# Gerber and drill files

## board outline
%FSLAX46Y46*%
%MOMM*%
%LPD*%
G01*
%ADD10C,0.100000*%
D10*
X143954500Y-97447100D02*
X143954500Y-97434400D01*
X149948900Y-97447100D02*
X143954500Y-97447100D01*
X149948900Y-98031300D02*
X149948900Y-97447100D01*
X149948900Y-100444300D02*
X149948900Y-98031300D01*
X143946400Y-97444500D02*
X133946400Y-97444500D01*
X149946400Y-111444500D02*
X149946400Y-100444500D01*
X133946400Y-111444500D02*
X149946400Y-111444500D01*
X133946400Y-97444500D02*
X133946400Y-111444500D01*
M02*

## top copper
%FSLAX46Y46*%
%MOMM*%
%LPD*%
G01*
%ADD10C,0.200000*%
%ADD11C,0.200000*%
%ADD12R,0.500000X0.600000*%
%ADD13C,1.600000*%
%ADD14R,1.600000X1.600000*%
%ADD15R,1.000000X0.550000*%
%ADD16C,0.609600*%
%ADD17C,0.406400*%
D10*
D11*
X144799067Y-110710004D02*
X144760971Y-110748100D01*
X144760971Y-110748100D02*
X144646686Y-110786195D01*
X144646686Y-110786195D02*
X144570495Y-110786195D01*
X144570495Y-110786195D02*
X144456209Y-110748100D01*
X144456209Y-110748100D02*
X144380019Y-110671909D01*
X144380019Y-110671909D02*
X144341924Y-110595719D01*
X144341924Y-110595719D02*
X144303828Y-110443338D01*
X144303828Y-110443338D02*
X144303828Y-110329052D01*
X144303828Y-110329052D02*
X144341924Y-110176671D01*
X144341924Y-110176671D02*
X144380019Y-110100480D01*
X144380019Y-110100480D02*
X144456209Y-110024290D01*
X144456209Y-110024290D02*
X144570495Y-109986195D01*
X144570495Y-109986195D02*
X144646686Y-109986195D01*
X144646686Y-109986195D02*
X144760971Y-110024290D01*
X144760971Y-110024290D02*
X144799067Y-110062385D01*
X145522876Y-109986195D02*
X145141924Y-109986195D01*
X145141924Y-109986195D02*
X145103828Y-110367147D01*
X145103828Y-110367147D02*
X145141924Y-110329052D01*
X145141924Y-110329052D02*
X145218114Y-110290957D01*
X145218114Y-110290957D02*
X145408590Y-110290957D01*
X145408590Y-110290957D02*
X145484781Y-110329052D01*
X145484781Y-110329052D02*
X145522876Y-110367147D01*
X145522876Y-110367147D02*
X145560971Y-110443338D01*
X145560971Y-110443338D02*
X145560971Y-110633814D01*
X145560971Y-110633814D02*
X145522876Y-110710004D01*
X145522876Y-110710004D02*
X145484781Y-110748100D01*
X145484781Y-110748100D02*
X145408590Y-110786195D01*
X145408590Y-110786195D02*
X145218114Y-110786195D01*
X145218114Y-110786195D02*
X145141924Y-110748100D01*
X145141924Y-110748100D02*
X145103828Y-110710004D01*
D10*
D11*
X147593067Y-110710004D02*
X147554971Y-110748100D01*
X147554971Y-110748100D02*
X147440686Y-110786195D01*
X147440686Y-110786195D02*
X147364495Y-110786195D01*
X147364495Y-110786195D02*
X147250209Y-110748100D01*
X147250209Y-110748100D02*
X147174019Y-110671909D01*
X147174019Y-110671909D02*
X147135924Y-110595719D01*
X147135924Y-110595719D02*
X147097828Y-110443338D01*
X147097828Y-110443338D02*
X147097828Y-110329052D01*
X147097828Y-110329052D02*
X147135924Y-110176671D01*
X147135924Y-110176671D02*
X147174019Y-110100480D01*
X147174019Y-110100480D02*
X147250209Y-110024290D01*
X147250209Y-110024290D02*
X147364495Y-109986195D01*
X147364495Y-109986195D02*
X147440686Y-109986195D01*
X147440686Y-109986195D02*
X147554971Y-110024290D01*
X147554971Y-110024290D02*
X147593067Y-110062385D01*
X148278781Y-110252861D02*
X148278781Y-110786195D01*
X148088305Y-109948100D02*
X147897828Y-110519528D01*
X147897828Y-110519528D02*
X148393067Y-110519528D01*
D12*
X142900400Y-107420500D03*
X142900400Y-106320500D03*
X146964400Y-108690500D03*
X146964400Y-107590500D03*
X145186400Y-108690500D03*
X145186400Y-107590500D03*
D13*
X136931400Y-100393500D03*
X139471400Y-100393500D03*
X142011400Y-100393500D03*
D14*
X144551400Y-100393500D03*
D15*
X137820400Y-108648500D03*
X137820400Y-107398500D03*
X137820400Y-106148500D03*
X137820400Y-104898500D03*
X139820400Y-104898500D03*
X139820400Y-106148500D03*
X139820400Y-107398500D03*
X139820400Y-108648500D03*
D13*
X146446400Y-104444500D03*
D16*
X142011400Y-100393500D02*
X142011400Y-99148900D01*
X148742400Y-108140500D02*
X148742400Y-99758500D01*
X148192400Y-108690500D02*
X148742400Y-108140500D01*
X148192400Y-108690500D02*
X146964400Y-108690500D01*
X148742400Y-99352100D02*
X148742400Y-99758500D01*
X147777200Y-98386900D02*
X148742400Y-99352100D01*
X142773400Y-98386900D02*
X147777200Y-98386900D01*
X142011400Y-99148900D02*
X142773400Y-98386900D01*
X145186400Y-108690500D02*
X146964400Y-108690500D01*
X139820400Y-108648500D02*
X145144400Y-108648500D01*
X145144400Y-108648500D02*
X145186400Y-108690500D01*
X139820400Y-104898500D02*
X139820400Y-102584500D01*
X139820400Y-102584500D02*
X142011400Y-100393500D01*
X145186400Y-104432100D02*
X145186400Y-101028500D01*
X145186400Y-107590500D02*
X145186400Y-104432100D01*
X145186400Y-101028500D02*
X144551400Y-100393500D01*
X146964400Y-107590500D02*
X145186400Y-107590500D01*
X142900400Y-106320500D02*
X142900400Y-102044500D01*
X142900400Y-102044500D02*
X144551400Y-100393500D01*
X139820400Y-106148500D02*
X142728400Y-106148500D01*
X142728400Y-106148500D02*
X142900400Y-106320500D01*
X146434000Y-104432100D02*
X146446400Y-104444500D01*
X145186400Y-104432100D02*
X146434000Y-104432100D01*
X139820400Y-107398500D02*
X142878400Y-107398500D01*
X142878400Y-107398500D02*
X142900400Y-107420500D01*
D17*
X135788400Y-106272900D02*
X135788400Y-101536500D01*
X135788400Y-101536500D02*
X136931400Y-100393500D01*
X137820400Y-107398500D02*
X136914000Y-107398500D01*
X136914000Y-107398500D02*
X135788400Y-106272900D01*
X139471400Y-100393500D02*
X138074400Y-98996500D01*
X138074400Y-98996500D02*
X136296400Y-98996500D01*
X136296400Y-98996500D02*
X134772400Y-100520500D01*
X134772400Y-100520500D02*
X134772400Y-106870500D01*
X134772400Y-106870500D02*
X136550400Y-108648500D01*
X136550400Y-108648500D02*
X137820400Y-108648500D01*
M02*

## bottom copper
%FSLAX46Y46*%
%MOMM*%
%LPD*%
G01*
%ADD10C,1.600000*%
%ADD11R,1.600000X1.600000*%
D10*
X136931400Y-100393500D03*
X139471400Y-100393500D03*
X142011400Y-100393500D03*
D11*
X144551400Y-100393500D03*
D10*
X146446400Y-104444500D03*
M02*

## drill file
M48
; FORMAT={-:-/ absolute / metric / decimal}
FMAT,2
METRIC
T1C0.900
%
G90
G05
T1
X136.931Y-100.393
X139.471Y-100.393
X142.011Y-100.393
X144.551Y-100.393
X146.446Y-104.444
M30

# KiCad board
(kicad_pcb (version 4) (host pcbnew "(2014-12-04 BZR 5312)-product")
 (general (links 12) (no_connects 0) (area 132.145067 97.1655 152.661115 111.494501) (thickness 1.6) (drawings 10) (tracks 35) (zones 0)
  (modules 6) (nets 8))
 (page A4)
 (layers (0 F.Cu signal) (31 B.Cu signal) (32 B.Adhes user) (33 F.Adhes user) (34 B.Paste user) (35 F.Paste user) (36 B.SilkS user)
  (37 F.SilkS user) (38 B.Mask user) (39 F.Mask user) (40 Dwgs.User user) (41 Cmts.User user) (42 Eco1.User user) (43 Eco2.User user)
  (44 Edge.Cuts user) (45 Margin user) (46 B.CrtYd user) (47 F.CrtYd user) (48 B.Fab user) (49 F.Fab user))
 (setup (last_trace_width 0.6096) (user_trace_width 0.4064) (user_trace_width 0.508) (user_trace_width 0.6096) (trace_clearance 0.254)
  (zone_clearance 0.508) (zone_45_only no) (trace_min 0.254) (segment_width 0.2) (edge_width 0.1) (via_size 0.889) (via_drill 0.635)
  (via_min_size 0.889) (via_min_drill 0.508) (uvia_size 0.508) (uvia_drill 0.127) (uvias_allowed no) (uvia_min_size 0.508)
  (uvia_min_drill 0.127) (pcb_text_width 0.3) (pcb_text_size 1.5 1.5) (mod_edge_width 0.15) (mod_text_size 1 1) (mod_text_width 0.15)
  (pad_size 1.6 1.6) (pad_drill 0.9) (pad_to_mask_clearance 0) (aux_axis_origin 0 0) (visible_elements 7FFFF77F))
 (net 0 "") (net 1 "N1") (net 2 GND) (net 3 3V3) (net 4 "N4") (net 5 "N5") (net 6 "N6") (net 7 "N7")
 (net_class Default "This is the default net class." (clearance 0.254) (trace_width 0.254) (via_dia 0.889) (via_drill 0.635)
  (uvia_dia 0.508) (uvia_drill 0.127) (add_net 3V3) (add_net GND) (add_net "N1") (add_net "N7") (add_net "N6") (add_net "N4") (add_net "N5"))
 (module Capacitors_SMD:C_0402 (layer F.Cu) (at 142.9004 106.8705 90)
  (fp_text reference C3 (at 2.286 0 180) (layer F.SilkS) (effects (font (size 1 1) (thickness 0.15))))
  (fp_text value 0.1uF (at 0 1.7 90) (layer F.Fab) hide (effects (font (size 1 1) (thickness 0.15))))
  (pad 1 smd rect (at -0.55 0 90) (size 0.6 0.5) (layers F.Cu F.Paste F.Mask) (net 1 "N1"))
  (pad 2 smd rect (at 0.55 0 90) (size 0.6 0.5) (layers F.Cu F.Paste F.Mask) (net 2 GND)))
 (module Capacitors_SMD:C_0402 (layer F.Cu) (at 146.9644 108.1405 90)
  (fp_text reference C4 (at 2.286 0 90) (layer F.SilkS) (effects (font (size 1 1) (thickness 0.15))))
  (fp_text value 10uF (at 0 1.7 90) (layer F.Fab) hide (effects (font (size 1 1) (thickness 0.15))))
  (pad 1 smd rect (at -0.55 0 90) (size 0.6 0.5) (layers F.Cu F.Paste F.Mask) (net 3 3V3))
  (pad 2 smd rect (at 0.55 0 90) (size 0.6 0.5) (layers F.Cu F.Paste F.Mask) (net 2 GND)))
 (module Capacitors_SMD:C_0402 (layer F.Cu) (at 145.1864 108.1405 90)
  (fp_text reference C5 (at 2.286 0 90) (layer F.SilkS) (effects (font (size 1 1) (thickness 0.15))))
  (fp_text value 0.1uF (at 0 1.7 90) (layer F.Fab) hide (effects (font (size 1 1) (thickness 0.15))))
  (pad 1 smd rect (at -0.55 0 90) (size 0.6 0.5) (layers F.Cu F.Paste F.Mask) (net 3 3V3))
  (pad 2 smd rect (at 0.55 0 90) (size 0.6 0.5) (layers F.Cu F.Paste F.Mask) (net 2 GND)))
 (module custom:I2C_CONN (layer F.Cu) (at 142.0114 100.3935)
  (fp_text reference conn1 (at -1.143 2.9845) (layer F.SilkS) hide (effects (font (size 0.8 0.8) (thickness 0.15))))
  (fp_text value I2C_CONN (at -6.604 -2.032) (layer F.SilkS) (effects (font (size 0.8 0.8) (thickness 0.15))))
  (pad 1 thru_hole circle (at -5.08 0) (size 1.6 1.6) (drill 0.9) (layers *.Cu *.Mask F.SilkS) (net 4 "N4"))
  (pad 2 thru_hole circle (at -2.54 0) (size 1.6 1.6) (drill 0.9) (layers *.Cu *.Mask F.SilkS) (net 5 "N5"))
  (pad 3 thru_hole circle (at 0 0) (size 1.6 1.6) (drill 0.9) (layers *.Cu *.Mask F.SilkS) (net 3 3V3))
  (pad 4 thru_hole rect (at 2.54 0) (size 1.6 1.6) (drill 0.9) (layers *.Cu *.Mask F.SilkS) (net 2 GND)))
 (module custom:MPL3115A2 (layer F.Cu) (at 137.8204 108.6485 180)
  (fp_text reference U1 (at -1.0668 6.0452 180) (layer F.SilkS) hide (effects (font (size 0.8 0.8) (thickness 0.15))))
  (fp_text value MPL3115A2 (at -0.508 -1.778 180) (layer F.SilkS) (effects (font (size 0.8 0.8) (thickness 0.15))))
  (pad 8 smd rect (at 0 0 180) (size 1 0.55) (layers F.Cu F.Paste F.Mask) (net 5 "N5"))
  (pad 7 smd rect (at 0 1.25 180) (size 1 0.55) (layers F.Cu F.Paste F.Mask) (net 4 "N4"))
  (pad 6 smd rect (at 0 2.5 180) (size 1 0.55) (layers F.Cu F.Paste F.Mask) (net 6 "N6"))
  (pad 5 smd rect (at 0 3.75 180) (size 1 0.55) (layers F.Cu F.Paste F.Mask) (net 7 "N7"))
  (pad 4 smd rect (at -2 3.75 180) (size 1 0.55) (layers F.Cu F.Paste F.Mask) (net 3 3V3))
  (pad 3 smd rect (at -2 2.5 180) (size 1 0.55) (layers F.Cu F.Paste F.Mask) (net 2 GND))
  (pad 2 smd rect (at -2 1.25 180) (size 1 0.55) (layers F.Cu F.Paste F.Mask) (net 1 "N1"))
  (pad 1 smd rect (at -2 0 180) (size 1 0.55) (layers F.Cu F.Paste F.Mask) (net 3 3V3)))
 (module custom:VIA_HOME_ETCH (layer F.Cu) (at 146.4464 104.4445)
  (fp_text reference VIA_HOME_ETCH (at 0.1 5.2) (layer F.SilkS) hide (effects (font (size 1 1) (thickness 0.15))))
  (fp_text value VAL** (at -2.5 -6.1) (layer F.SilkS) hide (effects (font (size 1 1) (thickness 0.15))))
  (pad 1 thru_hole circle (at 0 0) (size 1.6 1.6) (drill 0.9) (layers *.Cu *.Mask F.SilkS) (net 2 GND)))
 (gr_line (start 143.9545 97.4471) (end 143.9545 97.4344) (angle 90) (layer Edge.Cuts) (width 0.1))
 (gr_line (start 149.9489 97.4471) (end 143.9545 97.4471) (angle 90) (layer Edge.Cuts) (width 0.1))
 (gr_line (start 149.9489 98.0313) (end 149.9489 97.4471) (angle 90) (layer Edge.Cuts) (width 0.1))
 (gr_line (start 149.9489 100.4443) (end 149.9489 98.0313) (angle 90) (layer Edge.Cuts) (width 0.1))
 (gr_line (start 143.9464 97.4445) (end 133.9464 97.4445) (angle 90) (layer Edge.Cuts) (width 0.1))
 (gr_line (start 149.9464 111.4445) (end 149.9464 100.4445) (angle 90) (layer Edge.Cuts) (width 0.1))
 (gr_line (start 133.9464 111.4445) (end 149.9464 111.4445) (angle 90) (layer Edge.Cuts) (width 0.1))
 (gr_line (start 133.9464 97.4445) (end 133.9464 111.4445) (angle 90) (layer Edge.Cuts) (width 0.1))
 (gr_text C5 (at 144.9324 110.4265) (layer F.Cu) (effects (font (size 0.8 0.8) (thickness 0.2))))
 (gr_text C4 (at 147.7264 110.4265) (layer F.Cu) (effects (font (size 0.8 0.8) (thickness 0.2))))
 (segment (start 142.0114 100.3935) (end 142.0114 99.1489) (width 0.6096) (layer F.Cu) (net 3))
 (segment (start 148.7424 108.1405) (end 148.7424 99.7585) (width 0.6096) (layer F.Cu) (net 3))
 (segment (start 148.1924 108.6905) (end 148.7424 108.1405) (width 0.6096) (layer F.Cu) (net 3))
 (segment (start 148.1924 108.6905) (end 146.9644 108.6905) (width 0.6096) (layer F.Cu) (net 3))
 (segment (start 148.7424 99.3521) (end 148.7424 99.7585) (width 0.6096) (layer F.Cu) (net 3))
 (segment (start 147.7772 98.3869) (end 148.7424 99.3521) (width 0.6096) (layer F.Cu) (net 3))
 (segment (start 142.7734 98.3869) (end 147.7772 98.3869) (width 0.6096) (layer F.Cu) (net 3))
 (segment (start 142.0114 99.1489) (end 142.7734 98.3869) (width 0.6096) (layer F.Cu) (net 3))
 (segment (start 145.1864 108.6905) (end 146.9644 108.6905) (width 0.6096) (layer F.Cu) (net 3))
 (segment (start 139.8204 108.6485) (end 145.1444 108.6485) (width 0.6096) (layer F.Cu) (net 3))
 (segment (start 145.1444 108.6485) (end 145.1864 108.6905) (width 0.6096) (layer F.Cu) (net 3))
 (segment (start 139.8204 104.8985) (end 139.8204 102.5845) (width 0.6096) (layer F.Cu) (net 3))
 (segment (start 139.8204 102.5845) (end 142.0114 100.3935) (width 0.6096) (layer F.Cu) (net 3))
 (segment (start 145.1864 104.4321) (end 145.1864 101.0285) (width 0.6096) (layer F.Cu) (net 2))
 (segment (start 145.1864 107.5905) (end 145.1864 104.4321) (width 0.6096) (layer F.Cu) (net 2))
 (segment (start 145.1864 101.0285) (end 144.5514 100.3935) (width 0.6096) (layer F.Cu) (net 2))
 (segment (start 146.9644 107.5905) (end 145.1864 107.5905) (width 0.6096) (layer F.Cu) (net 2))
 (segment (start 142.9004 106.3205) (end 142.9004 102.0445) (width 0.6096) (layer F.Cu) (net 2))
 (segment (start 142.9004 102.0445) (end 144.5514 100.3935) (width 0.6096) (layer F.Cu) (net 2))
 (segment (start 139.8204 106.1485) (end 142.7284 106.1485) (width 0.6096) (layer F.Cu) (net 2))
 (segment (start 142.7284 106.1485) (end 142.9004 106.3205) (width 0.6096) (layer F.Cu) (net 2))
 (segment (start 146.434 104.4321) (end 146.4464 104.4445) (width 0.6096) (layer F.Cu) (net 2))
 (segment (start 145.1864 104.4321) (end 146.434 104.4321) (width 0.6096) (layer F.Cu) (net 2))
 (segment (start 139.8204 107.3985) (end 142.8784 107.3985) (width 0.6096) (layer F.Cu) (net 1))
 (segment (start 142.8784 107.3985) (end 142.9004 107.4205) (width 0.6096) (layer F.Cu) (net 1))
 (segment (start 135.7884 106.2729) (end 135.7884 101.5365) (width 0.4064) (layer F.Cu) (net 4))
 (segment (start 135.7884 101.5365) (end 136.9314 100.3935) (width 0.4064) (layer F.Cu) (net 4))
 (segment (start 137.8204 107.3985) (end 136.914 107.3985) (width 0.4064) (layer F.Cu) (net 4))
 (segment (start 136.914 107.3985) (end 135.7884 106.2729) (width 0.4064) (layer F.Cu) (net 4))
 (segment (start 139.4714 100.3935) (end 138.0744 98.9965) (width 0.4064) (layer F.Cu) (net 5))
 (segment (start 138.0744 98.9965) (end 136.2964 98.9965) (width 0.4064) (layer F.Cu) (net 5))
 (segment (start 136.2964 98.9965) (end 134.7724 100.5205) (width 0.4064) (layer F.Cu) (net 5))
 (segment (start 134.7724 100.5205) (end 134.7724 106.8705) (width 0.4064) (layer F.Cu) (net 5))
 (segment (start 134.7724 106.8705) (end 136.5504 108.6485) (width 0.4064) (layer F.Cu) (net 5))
 (segment (start 136.5504 108.6485) (end 137.8204 108.6485) (width 0.4064) (layer F.Cu) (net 5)))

